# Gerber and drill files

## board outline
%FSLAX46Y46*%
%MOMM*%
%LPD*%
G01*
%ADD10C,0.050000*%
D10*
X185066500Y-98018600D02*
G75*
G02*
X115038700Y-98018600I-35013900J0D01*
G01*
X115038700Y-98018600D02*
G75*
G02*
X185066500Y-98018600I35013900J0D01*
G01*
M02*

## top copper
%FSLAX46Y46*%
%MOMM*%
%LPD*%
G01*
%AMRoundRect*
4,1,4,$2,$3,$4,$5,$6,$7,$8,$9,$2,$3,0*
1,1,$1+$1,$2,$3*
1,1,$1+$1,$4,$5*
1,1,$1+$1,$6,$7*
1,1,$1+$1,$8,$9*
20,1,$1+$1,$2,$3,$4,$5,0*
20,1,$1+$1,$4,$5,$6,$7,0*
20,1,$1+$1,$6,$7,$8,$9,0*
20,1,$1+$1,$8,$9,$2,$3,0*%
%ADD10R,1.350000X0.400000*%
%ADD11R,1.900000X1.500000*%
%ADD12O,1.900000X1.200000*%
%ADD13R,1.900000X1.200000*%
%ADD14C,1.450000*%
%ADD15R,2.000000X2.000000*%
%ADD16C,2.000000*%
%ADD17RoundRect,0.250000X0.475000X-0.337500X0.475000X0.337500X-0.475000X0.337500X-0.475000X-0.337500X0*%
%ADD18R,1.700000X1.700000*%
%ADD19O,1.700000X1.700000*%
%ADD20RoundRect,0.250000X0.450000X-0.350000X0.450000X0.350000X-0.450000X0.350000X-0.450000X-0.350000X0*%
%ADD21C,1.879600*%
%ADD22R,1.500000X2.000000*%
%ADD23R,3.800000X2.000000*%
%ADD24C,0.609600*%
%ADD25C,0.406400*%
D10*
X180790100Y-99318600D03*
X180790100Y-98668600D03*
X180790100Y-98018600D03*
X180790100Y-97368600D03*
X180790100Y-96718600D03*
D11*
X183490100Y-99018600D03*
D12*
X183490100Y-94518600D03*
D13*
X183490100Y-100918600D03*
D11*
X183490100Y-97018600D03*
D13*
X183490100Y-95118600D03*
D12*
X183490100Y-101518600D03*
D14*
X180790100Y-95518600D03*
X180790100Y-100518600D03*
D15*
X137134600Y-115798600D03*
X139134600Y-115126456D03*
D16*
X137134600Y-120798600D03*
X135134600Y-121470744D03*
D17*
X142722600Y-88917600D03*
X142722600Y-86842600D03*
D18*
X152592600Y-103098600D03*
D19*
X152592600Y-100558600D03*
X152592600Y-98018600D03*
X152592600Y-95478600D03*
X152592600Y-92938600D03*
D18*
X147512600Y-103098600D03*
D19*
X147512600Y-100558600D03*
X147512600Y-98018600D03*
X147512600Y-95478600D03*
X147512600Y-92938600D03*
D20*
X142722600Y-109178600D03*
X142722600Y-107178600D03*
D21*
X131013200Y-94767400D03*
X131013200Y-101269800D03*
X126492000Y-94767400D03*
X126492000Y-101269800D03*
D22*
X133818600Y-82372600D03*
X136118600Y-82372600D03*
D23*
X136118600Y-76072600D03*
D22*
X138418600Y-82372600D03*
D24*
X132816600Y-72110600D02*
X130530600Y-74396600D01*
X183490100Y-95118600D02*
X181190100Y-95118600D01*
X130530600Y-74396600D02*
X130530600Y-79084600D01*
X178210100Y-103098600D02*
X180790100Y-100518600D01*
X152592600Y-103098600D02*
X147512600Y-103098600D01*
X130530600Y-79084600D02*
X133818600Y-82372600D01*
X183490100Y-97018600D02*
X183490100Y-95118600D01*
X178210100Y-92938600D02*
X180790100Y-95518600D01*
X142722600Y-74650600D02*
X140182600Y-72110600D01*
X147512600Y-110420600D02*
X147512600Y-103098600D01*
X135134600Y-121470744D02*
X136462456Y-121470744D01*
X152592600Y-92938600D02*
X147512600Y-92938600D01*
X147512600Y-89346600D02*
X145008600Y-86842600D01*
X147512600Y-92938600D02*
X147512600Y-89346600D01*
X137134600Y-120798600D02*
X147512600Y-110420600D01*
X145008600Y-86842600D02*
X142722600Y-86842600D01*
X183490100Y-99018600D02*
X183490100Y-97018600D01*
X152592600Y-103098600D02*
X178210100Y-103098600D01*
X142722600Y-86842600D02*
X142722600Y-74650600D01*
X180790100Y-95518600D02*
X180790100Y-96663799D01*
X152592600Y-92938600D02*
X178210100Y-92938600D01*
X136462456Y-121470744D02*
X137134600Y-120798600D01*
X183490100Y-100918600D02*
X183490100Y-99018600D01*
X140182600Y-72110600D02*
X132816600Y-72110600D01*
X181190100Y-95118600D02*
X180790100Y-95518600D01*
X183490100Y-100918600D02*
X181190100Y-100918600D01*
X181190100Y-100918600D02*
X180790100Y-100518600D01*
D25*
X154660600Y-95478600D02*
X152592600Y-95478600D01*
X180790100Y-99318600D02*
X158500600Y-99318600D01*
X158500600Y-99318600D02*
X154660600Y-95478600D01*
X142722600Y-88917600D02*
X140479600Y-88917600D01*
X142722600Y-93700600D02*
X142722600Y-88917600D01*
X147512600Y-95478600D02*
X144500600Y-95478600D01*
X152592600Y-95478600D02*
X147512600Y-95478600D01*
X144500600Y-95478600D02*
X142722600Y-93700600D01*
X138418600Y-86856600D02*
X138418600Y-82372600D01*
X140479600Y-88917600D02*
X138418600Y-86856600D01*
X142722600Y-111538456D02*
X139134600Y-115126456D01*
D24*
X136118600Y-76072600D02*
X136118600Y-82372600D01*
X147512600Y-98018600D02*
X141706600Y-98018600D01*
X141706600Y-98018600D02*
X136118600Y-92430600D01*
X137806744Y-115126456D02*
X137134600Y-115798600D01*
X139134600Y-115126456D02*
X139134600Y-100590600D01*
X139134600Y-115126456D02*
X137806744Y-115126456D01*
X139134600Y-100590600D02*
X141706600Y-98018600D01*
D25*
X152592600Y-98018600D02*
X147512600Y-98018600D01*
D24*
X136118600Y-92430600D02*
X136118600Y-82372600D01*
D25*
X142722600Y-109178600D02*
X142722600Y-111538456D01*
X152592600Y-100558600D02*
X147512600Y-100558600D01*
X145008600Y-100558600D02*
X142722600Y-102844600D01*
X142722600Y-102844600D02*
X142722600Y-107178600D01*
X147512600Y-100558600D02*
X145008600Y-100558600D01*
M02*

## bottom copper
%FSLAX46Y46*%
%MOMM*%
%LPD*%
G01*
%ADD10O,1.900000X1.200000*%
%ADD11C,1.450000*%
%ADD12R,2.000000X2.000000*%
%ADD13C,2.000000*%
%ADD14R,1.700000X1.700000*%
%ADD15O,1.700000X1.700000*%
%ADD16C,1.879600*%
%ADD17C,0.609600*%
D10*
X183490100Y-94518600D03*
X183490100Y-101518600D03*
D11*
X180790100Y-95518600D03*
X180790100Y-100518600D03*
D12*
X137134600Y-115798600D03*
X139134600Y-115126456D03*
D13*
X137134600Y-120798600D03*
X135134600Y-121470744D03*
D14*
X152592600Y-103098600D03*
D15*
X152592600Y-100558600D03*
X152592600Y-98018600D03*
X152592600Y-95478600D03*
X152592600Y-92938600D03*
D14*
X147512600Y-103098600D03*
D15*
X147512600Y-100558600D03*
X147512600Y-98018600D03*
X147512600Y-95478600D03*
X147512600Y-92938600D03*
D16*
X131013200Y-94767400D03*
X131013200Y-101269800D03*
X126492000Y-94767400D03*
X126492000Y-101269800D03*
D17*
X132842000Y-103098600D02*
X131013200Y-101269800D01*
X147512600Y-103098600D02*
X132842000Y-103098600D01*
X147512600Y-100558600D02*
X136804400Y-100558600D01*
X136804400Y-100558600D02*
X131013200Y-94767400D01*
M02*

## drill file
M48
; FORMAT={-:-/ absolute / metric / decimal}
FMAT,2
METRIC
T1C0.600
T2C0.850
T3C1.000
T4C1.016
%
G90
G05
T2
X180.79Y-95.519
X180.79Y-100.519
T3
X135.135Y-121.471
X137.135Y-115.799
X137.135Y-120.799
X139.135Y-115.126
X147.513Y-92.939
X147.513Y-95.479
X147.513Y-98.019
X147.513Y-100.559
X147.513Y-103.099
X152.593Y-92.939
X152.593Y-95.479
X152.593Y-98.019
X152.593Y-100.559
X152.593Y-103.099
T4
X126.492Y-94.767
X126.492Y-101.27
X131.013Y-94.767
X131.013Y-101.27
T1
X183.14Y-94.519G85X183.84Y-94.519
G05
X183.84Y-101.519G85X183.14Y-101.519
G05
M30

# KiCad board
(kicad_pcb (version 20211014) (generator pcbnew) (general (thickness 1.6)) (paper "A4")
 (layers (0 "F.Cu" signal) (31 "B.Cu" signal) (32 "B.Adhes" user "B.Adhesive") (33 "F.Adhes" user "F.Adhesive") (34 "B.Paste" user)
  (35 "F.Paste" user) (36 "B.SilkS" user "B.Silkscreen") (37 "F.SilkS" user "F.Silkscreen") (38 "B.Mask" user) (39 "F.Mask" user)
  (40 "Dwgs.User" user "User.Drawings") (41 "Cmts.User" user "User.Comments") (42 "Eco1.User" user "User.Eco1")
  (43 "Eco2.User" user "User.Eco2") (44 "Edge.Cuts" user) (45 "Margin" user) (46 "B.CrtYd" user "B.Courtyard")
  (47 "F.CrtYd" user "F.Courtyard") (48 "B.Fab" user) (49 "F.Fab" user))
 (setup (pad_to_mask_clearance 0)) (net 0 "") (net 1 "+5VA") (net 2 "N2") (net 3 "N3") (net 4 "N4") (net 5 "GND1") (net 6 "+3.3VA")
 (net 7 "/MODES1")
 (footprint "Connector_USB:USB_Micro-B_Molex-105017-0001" (layer "F.Cu") (at 182.2526 98.0186 90)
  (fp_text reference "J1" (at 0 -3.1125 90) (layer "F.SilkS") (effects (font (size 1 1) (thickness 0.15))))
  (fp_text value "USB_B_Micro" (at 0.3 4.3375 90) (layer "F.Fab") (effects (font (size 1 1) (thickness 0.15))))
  (pad "1" smd rect locked (at -1.3 -1.4625 90) (size 0.4 1.35) (layers "F.Cu" "F.Paste" "F.Mask") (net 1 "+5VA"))
  (pad "2" smd rect locked (at -0.65 -1.4625 90) (size 0.4 1.35) (layers "F.Cu" "F.Paste" "F.Mask") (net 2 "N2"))
  (pad "3" smd rect locked (at 0 -1.4625 90) (size 0.4 1.35) (layers "F.Cu" "F.Paste" "F.Mask") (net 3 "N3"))
  (pad "4" smd rect locked (at 0.65 -1.4625 90) (size 0.4 1.35) (layers "F.Cu" "F.Paste" "F.Mask") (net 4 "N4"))
  (pad "5" smd rect locked (at 1.3 -1.4625 90) (size 0.4 1.35) (layers "F.Cu" "F.Paste" "F.Mask") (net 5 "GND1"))
  (pad "6" smd rect locked (at -1 1.2375 90) (size 1.5 1.9) (layers "F.Cu" "F.Paste" "F.Mask") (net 5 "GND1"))
  (pad "6" thru_hole oval locked (at 3.5 1.2375 90) (size 1.2 1.9) (drill oval 0.6 1.3) (layers *.Cu *.Mask) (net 5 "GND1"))
  (pad "6" smd rect locked (at -2.9 1.2375 90) (size 1.2 1.9) (layers "F.Cu" "F.Mask") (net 5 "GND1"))
  (pad "6" smd rect locked (at 1 1.2375 90) (size 1.5 1.9) (layers "F.Cu" "F.Paste" "F.Mask") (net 5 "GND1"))
  (pad "6" smd rect locked (at 2.9 1.2375 90) (size 1.2 1.9) (layers "F.Cu" "F.Mask") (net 5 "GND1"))
  (pad "6" thru_hole oval locked (at -3.5 1.2375 270) (size 1.2 1.9) (drill oval 0.6 1.3) (layers *.Cu *.Mask) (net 5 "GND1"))
  (pad "6" thru_hole circle locked (at 2.5 -1.4625 90) (size 1.45 1.45) (drill 0.85) (layers *.Cu *.Mask) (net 5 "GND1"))
  (pad "6" thru_hole circle locked (at -2.5 -1.4625 90) (size 1.45 1.45) (drill 0.85) (layers *.Cu *.Mask) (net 5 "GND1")))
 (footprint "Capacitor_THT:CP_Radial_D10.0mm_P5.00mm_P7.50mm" (layer "F.Cu") (at 137.1346 115.7986 -90)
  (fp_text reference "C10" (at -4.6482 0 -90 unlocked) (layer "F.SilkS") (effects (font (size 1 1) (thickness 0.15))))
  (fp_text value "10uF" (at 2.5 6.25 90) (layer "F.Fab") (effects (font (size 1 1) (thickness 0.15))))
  (pad "1" thru_hole rect locked (at 0 0 270) (size 2 2) (drill 1) (layers *.Cu *.Mask) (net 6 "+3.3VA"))
  (pad "1" thru_hole rect locked (at -0.672144 -2 270) (size 2 2) (drill 1) (layers *.Cu *.Mask) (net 6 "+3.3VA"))
  (pad "2" thru_hole circle locked (at 5 0 270) (size 2 2) (drill 1) (layers *.Cu *.Mask) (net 5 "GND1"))
  (pad "2" thru_hole circle locked (at 5.672144 2 270) (size 2 2) (drill 1) (layers *.Cu *.Mask) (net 5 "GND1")))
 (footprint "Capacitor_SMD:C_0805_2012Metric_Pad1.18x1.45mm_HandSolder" (layer "F.Cu") (at 142.7226 87.8801 90)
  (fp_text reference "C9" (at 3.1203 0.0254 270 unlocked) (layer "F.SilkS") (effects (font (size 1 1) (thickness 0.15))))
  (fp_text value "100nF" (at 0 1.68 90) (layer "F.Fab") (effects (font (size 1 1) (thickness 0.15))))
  (pad "1" smd roundrect locked (at -1.0375 0 90) (size 1.175 1.45) (layers "F.Cu" "F.Paste" "F.Mask") (roundrect_rratio 0.212766)
   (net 1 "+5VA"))
  (pad "2" smd roundrect locked (at 1.0375 0 90) (size 1.175 1.45) (layers "F.Cu" "F.Paste" "F.Mask") (roundrect_rratio 0.212766)
   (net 5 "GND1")))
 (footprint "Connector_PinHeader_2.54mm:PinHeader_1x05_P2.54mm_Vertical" (layer "F.Cu") (at 152.5926 103.0986 180)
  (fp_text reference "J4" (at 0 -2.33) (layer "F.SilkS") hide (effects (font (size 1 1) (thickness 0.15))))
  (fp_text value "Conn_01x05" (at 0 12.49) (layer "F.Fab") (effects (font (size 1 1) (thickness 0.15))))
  (pad "1" thru_hole rect locked (at 0 0 180) (size 1.7 1.7) (drill 1) (layers *.Cu *.Mask) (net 5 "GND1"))
  (pad "2" thru_hole oval locked (at 0 2.54 180) (size 1.7 1.7) (drill 1) (layers *.Cu *.Mask) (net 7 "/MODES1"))
  (pad "3" thru_hole oval locked (at 0 5.08 180) (size 1.7 1.7) (drill 1) (layers *.Cu *.Mask) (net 6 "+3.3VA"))
  (pad "4" thru_hole oval locked (at 0 7.62 180) (size 1.7 1.7) (drill 1) (layers *.Cu *.Mask) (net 1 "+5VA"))
  (pad "5" thru_hole oval locked (at 0 10.16 180) (size 1.7 1.7) (drill 1) (layers *.Cu *.Mask) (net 5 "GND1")))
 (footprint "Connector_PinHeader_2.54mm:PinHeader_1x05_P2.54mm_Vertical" (layer "F.Cu") (at 147.5126 103.0986 180)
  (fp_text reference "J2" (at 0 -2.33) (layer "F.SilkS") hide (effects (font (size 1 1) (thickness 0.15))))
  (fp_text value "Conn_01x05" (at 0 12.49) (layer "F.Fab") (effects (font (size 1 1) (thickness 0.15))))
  (pad "1" thru_hole rect locked (at 0 0 180) (size 1.7 1.7) (drill 1) (layers *.Cu *.Mask) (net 5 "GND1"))
  (pad "2" thru_hole oval locked (at 0 2.54 180) (size 1.7 1.7) (drill 1) (layers *.Cu *.Mask) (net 7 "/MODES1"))
  (pad "3" thru_hole oval locked (at 0 5.08 180) (size 1.7 1.7) (drill 1) (layers *.Cu *.Mask) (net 6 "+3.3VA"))
  (pad "4" thru_hole oval locked (at 0 7.62 180) (size 1.7 1.7) (drill 1) (layers *.Cu *.Mask) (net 1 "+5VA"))
  (pad "5" thru_hole oval locked (at 0 10.16 180) (size 1.7 1.7) (drill 1) (layers *.Cu *.Mask) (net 5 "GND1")))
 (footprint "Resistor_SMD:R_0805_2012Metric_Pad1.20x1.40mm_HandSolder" (layer "F.Cu") (at 142.7226 108.1786 90)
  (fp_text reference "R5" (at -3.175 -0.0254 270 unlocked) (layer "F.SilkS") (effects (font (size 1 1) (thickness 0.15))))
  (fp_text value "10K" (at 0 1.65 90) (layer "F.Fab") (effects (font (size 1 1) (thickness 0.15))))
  (pad "1" smd roundrect locked (at -1 0 90) (size 1.2 1.4) (layers "F.Cu" "F.Paste" "F.Mask") (roundrect_rratio 0.208333) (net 6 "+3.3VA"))
  (pad "2" smd roundrect locked (at 1 0 90) (size 1.2 1.4) (layers "F.Cu" "F.Paste" "F.Mask") (roundrect_rratio 0.208333) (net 7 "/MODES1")))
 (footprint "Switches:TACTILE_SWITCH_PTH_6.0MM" (layer "F.Cu") (at 128.7526 98.0186 -90)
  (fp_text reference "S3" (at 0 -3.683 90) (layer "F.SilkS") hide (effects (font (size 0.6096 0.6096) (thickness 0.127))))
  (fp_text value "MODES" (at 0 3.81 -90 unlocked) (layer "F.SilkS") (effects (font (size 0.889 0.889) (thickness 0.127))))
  (pad "1" thru_hole circle locked (at -3.2512 -2.2606 270) (size 1.8796 1.8796) (drill 1.016) (layers *.Cu *.Mask) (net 7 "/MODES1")
   (solder_mask_margin 0.1016))
  (pad "2" thru_hole circle locked (at 3.2512 -2.2606 270) (size 1.8796 1.8796) (drill 1.016) (layers *.Cu *.Mask) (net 5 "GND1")
   (solder_mask_margin 0.1016))
  (pad "3" thru_hole circle locked (at -3.2512 2.2606 270) (size 1.8796 1.8796) (drill 1.016) (layers *.Cu *.Mask)
   (solder_mask_margin 0.1016))
  (pad "4" thru_hole circle locked (at 3.2512 2.2606 270) (size 1.8796 1.8796) (drill 1.016) (layers *.Cu *.Mask)
   (solder_mask_margin 0.1016)))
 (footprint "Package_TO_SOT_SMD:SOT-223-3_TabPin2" (layer "F.Cu") (at 136.1186 79.2226 90)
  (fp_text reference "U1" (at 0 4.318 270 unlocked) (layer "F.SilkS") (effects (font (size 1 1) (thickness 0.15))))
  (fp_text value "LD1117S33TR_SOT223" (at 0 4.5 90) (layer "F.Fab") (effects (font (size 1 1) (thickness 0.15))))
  (pad "1" smd rect locked (at -3.15 -2.3 90) (size 2 1.5) (layers "F.Cu" "F.Paste" "F.Mask") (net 5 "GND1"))
  (pad "2" smd rect locked (at -3.15 0 90) (size 2 1.5) (layers "F.Cu" "F.Paste" "F.Mask") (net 6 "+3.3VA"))
  (pad "2" smd rect locked (at 3.15 0 90) (size 2 3.8) (layers "F.Cu" "F.Paste" "F.Mask") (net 6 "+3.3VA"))
  (pad "3" smd rect locked (at -3.15 2.3 90) (size 2 1.5) (layers "F.Cu" "F.Paste" "F.Mask") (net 1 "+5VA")))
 (gr_circle (center 150.0526 98.0186) (end 185.0665 98.0186) (layer "Edge.Cuts") (width 0.05) (fill none))
 (segment (start 132.8166 72.1106) (end 130.5306 74.3966) (width 0.6096) (layer "F.Cu") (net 5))
 (segment (start 183.4901 95.1186) (end 181.1901 95.1186) (width 0.6096) (layer "F.Cu") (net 5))
 (segment (start 130.5306 74.3966) (end 130.5306 79.0846) (width 0.6096) (layer "F.Cu") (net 5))
 (segment (start 178.2101 103.0986) (end 180.7901 100.5186) (width 0.6096) (layer "F.Cu") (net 5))
 (segment (start 152.5926 103.0986) (end 147.5126 103.0986) (width 0.6096) (layer "F.Cu") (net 5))
 (segment (start 130.5306 79.0846) (end 133.8186 82.3726) (width 0.6096) (layer "F.Cu") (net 5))
 (segment (start 183.4901 97.0186) (end 183.4901 95.1186) (width 0.6096) (layer "F.Cu") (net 5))
 (segment (start 178.2101 92.9386) (end 180.7901 95.5186) (width 0.6096) (layer "F.Cu") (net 5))
 (segment (start 142.7226 74.6506) (end 140.1826 72.1106) (width 0.6096) (layer "F.Cu") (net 5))
 (segment (start 147.5126 110.4206) (end 147.5126 103.0986) (width 0.6096) (layer "F.Cu") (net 5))
 (segment (start 135.1346 121.470744) (end 136.462456 121.470744) (width 0.6096) (layer "F.Cu") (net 5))
 (segment (start 152.5926 92.9386) (end 147.5126 92.9386) (width 0.6096) (layer "F.Cu") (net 5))
 (segment (start 147.5126 89.3466) (end 145.0086 86.8426) (width 0.6096) (layer "F.Cu") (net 5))
 (segment (start 147.5126 92.9386) (end 147.5126 89.3466) (width 0.6096) (layer "F.Cu") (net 5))
 (segment (start 137.1346 120.7986) (end 147.5126 110.4206) (width 0.6096) (layer "F.Cu") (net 5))
 (segment (start 145.0086 86.8426) (end 142.7226 86.8426) (width 0.6096) (layer "F.Cu") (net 5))
 (segment (start 183.4901 99.0186) (end 183.4901 97.0186) (width 0.6096) (layer "F.Cu") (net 5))
 (segment (start 152.5926 103.0986) (end 178.2101 103.0986) (width 0.6096) (layer "F.Cu") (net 5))
 (segment (start 142.7226 86.8426) (end 142.7226 74.6506) (width 0.6096) (layer "F.Cu") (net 5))
 (segment (start 180.7901 95.5186) (end 180.7901 96.663799) (width 0.6096) (layer "F.Cu") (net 5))
 (segment (start 152.5926 92.9386) (end 178.2101 92.9386) (width 0.6096) (layer "F.Cu") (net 5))
 (segment (start 136.462456 121.470744) (end 137.1346 120.7986) (width 0.6096) (layer "F.Cu") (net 5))
 (segment (start 183.4901 100.9186) (end 183.4901 99.0186) (width 0.6096) (layer "F.Cu") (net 5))
 (segment (start 140.1826 72.1106) (end 132.8166 72.1106) (width 0.6096) (layer "F.Cu") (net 5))
 (segment (start 181.1901 95.1186) (end 180.7901 95.5186) (width 0.6096) (layer "F.Cu") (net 5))
 (segment (start 183.4901 100.9186) (end 181.1901 100.9186) (width 0.6096) (layer "F.Cu") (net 5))
 (segment (start 181.1901 100.9186) (end 180.7901 100.5186) (width 0.6096) (layer "F.Cu") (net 5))
 (segment (start 132.842 103.0986) (end 131.0132 101.2698) (width 0.6096) (layer "B.Cu") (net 5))
 (segment (start 147.5126 103.0986) (end 132.842 103.0986) (width 0.6096) (layer "B.Cu") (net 5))
 (segment (start 154.6606 95.4786) (end 152.5926 95.4786) (width 0.4064) (layer "F.Cu") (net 1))
 (segment (start 180.7901 99.3186) (end 158.5006 99.3186) (width 0.4064) (layer "F.Cu") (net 1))
 (segment (start 158.5006 99.3186) (end 154.6606 95.4786) (width 0.4064) (layer "F.Cu") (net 1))
 (segment (start 142.7226 88.9176) (end 140.4796 88.9176) (width 0.4064) (layer "F.Cu") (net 1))
 (segment (start 142.7226 93.7006) (end 142.7226 88.9176) (width 0.4064) (layer "F.Cu") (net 1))
 (segment (start 147.5126 95.4786) (end 144.5006 95.4786) (width 0.4064) (layer "F.Cu") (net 1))
 (segment (start 152.5926 95.4786) (end 147.5126 95.4786) (width 0.4064) (layer "F.Cu") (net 1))
 (segment (start 144.5006 95.4786) (end 142.7226 93.7006) (width 0.4064) (layer "F.Cu") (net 1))
 (segment (start 138.4186 86.8566) (end 138.4186 82.3726) (width 0.4064) (layer "F.Cu") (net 1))
 (segment (start 140.4796 88.9176) (end 138.4186 86.8566) (width 0.4064) (layer "F.Cu") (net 1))
 (segment (start 142.7226 111.538456) (end 139.1346 115.126456) (width 0.4064) (layer "F.Cu") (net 6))
 (segment (start 136.1186 76.0726) (end 136.1186 82.3726) (width 0.6096) (layer "F.Cu") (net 6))
 (segment (start 147.5126 98.0186) (end 141.7066 98.0186) (width 0.6096) (layer "F.Cu") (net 6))
 (segment (start 141.7066 98.0186) (end 136.1186 92.4306) (width 0.6096) (layer "F.Cu") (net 6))
 (segment (start 137.806744 115.126456) (end 137.1346 115.7986) (width 0.6096) (layer "F.Cu") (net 6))
 (segment (start 139.1346 115.126456) (end 139.1346 100.5906) (width 0.6096) (layer "F.Cu") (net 6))
 (segment (start 139.1346 115.126456) (end 137.806744 115.126456) (width 0.6096) (layer "F.Cu") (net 6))
 (segment (start 139.1346 100.5906) (end 141.7066 98.0186) (width 0.6096) (layer "F.Cu") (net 6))
 (segment (start 152.5926 98.0186) (end 147.5126 98.0186) (width 0.4064) (layer "F.Cu") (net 6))
 (segment (start 136.1186 92.4306) (end 136.1186 82.3726) (width 0.6096) (layer "F.Cu") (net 6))
 (segment (start 142.7226 109.1786) (end 142.7226 111.538456) (width 0.4064) (layer "F.Cu") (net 6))
 (segment (start 152.5926 100.5586) (end 147.5126 100.5586) (width 0.4064) (layer "F.Cu") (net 7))
 (segment (start 145.0086 100.5586) (end 142.7226 102.8446) (width 0.4064) (layer "F.Cu") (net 7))
 (segment (start 142.7226 102.8446) (end 142.7226 107.1786) (width 0.4064) (layer "F.Cu") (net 7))
 (segment (start 147.5126 100.5586) (end 145.0086 100.5586) (width 0.4064) (layer "F.Cu") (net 7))
 (segment (start 147.5126 100.5586) (end 136.8044 100.5586) (width 0.6096) (layer "B.Cu") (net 7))
 (segment (start 136.8044 100.5586) (end 131.0132 94.7674) (width 0.6096) (layer "B.Cu") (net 7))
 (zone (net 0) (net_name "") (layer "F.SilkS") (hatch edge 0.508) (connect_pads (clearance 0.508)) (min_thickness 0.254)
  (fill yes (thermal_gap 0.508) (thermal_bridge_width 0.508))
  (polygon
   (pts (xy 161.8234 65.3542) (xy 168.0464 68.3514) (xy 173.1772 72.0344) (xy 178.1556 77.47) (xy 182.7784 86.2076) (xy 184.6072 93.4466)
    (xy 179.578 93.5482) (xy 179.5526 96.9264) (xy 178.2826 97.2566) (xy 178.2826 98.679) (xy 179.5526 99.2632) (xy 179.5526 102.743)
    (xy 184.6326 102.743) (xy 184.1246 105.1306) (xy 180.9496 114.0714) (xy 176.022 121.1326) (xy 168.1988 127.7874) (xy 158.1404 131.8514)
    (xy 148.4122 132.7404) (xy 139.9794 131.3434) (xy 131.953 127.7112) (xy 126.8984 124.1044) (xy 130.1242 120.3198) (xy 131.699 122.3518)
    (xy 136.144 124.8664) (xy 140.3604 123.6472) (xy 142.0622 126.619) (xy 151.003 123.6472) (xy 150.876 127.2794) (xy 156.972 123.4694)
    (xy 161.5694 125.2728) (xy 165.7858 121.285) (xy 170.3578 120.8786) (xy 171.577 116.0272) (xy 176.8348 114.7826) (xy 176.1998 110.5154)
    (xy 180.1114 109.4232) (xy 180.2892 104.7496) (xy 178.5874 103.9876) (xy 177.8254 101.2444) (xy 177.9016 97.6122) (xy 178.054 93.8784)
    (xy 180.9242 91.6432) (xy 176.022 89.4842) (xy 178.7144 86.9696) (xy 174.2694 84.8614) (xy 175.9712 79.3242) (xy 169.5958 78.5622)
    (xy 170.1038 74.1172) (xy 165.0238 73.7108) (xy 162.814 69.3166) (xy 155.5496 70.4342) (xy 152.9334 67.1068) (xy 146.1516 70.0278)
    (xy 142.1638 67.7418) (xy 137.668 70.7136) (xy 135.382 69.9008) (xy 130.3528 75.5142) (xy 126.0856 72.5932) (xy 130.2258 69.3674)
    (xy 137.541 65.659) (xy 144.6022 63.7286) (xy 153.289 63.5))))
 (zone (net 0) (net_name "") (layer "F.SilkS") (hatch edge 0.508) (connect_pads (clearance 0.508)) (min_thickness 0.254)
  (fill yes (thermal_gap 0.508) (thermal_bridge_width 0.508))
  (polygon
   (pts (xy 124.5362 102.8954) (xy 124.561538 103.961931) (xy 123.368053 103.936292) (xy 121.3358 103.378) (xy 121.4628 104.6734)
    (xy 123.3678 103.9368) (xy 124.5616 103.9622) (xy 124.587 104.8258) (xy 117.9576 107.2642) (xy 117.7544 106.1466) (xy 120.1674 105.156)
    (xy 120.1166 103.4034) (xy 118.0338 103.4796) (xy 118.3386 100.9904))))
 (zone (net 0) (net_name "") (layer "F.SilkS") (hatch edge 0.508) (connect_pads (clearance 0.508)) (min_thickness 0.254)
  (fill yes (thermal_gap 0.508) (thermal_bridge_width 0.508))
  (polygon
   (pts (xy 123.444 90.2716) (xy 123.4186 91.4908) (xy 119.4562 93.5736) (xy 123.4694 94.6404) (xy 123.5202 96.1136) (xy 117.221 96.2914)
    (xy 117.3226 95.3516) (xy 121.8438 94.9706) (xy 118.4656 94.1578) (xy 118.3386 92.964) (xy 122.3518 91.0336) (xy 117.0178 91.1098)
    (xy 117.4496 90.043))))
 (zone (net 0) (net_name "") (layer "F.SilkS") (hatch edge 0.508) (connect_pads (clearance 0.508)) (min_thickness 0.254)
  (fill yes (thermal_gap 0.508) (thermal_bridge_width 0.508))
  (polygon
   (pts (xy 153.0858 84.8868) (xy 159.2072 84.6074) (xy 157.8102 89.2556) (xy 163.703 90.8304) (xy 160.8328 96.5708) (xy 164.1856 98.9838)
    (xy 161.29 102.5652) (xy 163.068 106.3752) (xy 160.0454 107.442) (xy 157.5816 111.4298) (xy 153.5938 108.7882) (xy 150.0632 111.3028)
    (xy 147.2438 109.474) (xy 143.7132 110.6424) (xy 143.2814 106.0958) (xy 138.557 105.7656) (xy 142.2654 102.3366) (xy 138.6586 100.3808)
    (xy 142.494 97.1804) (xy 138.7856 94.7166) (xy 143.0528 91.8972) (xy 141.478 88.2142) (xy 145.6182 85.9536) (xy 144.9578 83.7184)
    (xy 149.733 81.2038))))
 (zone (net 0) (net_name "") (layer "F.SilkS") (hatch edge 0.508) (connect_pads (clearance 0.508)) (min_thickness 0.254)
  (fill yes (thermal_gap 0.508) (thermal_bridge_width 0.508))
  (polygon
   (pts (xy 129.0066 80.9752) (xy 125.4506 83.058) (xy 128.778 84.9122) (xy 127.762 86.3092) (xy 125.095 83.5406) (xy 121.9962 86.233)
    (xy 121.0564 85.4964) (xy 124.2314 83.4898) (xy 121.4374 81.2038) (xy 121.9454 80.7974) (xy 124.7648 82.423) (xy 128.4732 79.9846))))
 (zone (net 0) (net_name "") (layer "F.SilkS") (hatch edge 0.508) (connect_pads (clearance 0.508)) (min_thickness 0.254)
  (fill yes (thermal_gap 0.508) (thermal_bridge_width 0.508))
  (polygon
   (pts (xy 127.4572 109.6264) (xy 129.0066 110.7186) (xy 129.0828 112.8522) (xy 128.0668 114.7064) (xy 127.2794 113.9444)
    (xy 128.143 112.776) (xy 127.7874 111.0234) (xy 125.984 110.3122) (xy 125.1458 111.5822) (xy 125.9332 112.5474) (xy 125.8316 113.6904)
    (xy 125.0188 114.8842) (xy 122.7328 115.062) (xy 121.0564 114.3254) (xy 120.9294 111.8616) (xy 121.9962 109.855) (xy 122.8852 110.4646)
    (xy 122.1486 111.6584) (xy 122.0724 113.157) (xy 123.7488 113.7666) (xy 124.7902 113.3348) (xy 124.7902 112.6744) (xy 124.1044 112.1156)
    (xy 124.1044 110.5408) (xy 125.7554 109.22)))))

